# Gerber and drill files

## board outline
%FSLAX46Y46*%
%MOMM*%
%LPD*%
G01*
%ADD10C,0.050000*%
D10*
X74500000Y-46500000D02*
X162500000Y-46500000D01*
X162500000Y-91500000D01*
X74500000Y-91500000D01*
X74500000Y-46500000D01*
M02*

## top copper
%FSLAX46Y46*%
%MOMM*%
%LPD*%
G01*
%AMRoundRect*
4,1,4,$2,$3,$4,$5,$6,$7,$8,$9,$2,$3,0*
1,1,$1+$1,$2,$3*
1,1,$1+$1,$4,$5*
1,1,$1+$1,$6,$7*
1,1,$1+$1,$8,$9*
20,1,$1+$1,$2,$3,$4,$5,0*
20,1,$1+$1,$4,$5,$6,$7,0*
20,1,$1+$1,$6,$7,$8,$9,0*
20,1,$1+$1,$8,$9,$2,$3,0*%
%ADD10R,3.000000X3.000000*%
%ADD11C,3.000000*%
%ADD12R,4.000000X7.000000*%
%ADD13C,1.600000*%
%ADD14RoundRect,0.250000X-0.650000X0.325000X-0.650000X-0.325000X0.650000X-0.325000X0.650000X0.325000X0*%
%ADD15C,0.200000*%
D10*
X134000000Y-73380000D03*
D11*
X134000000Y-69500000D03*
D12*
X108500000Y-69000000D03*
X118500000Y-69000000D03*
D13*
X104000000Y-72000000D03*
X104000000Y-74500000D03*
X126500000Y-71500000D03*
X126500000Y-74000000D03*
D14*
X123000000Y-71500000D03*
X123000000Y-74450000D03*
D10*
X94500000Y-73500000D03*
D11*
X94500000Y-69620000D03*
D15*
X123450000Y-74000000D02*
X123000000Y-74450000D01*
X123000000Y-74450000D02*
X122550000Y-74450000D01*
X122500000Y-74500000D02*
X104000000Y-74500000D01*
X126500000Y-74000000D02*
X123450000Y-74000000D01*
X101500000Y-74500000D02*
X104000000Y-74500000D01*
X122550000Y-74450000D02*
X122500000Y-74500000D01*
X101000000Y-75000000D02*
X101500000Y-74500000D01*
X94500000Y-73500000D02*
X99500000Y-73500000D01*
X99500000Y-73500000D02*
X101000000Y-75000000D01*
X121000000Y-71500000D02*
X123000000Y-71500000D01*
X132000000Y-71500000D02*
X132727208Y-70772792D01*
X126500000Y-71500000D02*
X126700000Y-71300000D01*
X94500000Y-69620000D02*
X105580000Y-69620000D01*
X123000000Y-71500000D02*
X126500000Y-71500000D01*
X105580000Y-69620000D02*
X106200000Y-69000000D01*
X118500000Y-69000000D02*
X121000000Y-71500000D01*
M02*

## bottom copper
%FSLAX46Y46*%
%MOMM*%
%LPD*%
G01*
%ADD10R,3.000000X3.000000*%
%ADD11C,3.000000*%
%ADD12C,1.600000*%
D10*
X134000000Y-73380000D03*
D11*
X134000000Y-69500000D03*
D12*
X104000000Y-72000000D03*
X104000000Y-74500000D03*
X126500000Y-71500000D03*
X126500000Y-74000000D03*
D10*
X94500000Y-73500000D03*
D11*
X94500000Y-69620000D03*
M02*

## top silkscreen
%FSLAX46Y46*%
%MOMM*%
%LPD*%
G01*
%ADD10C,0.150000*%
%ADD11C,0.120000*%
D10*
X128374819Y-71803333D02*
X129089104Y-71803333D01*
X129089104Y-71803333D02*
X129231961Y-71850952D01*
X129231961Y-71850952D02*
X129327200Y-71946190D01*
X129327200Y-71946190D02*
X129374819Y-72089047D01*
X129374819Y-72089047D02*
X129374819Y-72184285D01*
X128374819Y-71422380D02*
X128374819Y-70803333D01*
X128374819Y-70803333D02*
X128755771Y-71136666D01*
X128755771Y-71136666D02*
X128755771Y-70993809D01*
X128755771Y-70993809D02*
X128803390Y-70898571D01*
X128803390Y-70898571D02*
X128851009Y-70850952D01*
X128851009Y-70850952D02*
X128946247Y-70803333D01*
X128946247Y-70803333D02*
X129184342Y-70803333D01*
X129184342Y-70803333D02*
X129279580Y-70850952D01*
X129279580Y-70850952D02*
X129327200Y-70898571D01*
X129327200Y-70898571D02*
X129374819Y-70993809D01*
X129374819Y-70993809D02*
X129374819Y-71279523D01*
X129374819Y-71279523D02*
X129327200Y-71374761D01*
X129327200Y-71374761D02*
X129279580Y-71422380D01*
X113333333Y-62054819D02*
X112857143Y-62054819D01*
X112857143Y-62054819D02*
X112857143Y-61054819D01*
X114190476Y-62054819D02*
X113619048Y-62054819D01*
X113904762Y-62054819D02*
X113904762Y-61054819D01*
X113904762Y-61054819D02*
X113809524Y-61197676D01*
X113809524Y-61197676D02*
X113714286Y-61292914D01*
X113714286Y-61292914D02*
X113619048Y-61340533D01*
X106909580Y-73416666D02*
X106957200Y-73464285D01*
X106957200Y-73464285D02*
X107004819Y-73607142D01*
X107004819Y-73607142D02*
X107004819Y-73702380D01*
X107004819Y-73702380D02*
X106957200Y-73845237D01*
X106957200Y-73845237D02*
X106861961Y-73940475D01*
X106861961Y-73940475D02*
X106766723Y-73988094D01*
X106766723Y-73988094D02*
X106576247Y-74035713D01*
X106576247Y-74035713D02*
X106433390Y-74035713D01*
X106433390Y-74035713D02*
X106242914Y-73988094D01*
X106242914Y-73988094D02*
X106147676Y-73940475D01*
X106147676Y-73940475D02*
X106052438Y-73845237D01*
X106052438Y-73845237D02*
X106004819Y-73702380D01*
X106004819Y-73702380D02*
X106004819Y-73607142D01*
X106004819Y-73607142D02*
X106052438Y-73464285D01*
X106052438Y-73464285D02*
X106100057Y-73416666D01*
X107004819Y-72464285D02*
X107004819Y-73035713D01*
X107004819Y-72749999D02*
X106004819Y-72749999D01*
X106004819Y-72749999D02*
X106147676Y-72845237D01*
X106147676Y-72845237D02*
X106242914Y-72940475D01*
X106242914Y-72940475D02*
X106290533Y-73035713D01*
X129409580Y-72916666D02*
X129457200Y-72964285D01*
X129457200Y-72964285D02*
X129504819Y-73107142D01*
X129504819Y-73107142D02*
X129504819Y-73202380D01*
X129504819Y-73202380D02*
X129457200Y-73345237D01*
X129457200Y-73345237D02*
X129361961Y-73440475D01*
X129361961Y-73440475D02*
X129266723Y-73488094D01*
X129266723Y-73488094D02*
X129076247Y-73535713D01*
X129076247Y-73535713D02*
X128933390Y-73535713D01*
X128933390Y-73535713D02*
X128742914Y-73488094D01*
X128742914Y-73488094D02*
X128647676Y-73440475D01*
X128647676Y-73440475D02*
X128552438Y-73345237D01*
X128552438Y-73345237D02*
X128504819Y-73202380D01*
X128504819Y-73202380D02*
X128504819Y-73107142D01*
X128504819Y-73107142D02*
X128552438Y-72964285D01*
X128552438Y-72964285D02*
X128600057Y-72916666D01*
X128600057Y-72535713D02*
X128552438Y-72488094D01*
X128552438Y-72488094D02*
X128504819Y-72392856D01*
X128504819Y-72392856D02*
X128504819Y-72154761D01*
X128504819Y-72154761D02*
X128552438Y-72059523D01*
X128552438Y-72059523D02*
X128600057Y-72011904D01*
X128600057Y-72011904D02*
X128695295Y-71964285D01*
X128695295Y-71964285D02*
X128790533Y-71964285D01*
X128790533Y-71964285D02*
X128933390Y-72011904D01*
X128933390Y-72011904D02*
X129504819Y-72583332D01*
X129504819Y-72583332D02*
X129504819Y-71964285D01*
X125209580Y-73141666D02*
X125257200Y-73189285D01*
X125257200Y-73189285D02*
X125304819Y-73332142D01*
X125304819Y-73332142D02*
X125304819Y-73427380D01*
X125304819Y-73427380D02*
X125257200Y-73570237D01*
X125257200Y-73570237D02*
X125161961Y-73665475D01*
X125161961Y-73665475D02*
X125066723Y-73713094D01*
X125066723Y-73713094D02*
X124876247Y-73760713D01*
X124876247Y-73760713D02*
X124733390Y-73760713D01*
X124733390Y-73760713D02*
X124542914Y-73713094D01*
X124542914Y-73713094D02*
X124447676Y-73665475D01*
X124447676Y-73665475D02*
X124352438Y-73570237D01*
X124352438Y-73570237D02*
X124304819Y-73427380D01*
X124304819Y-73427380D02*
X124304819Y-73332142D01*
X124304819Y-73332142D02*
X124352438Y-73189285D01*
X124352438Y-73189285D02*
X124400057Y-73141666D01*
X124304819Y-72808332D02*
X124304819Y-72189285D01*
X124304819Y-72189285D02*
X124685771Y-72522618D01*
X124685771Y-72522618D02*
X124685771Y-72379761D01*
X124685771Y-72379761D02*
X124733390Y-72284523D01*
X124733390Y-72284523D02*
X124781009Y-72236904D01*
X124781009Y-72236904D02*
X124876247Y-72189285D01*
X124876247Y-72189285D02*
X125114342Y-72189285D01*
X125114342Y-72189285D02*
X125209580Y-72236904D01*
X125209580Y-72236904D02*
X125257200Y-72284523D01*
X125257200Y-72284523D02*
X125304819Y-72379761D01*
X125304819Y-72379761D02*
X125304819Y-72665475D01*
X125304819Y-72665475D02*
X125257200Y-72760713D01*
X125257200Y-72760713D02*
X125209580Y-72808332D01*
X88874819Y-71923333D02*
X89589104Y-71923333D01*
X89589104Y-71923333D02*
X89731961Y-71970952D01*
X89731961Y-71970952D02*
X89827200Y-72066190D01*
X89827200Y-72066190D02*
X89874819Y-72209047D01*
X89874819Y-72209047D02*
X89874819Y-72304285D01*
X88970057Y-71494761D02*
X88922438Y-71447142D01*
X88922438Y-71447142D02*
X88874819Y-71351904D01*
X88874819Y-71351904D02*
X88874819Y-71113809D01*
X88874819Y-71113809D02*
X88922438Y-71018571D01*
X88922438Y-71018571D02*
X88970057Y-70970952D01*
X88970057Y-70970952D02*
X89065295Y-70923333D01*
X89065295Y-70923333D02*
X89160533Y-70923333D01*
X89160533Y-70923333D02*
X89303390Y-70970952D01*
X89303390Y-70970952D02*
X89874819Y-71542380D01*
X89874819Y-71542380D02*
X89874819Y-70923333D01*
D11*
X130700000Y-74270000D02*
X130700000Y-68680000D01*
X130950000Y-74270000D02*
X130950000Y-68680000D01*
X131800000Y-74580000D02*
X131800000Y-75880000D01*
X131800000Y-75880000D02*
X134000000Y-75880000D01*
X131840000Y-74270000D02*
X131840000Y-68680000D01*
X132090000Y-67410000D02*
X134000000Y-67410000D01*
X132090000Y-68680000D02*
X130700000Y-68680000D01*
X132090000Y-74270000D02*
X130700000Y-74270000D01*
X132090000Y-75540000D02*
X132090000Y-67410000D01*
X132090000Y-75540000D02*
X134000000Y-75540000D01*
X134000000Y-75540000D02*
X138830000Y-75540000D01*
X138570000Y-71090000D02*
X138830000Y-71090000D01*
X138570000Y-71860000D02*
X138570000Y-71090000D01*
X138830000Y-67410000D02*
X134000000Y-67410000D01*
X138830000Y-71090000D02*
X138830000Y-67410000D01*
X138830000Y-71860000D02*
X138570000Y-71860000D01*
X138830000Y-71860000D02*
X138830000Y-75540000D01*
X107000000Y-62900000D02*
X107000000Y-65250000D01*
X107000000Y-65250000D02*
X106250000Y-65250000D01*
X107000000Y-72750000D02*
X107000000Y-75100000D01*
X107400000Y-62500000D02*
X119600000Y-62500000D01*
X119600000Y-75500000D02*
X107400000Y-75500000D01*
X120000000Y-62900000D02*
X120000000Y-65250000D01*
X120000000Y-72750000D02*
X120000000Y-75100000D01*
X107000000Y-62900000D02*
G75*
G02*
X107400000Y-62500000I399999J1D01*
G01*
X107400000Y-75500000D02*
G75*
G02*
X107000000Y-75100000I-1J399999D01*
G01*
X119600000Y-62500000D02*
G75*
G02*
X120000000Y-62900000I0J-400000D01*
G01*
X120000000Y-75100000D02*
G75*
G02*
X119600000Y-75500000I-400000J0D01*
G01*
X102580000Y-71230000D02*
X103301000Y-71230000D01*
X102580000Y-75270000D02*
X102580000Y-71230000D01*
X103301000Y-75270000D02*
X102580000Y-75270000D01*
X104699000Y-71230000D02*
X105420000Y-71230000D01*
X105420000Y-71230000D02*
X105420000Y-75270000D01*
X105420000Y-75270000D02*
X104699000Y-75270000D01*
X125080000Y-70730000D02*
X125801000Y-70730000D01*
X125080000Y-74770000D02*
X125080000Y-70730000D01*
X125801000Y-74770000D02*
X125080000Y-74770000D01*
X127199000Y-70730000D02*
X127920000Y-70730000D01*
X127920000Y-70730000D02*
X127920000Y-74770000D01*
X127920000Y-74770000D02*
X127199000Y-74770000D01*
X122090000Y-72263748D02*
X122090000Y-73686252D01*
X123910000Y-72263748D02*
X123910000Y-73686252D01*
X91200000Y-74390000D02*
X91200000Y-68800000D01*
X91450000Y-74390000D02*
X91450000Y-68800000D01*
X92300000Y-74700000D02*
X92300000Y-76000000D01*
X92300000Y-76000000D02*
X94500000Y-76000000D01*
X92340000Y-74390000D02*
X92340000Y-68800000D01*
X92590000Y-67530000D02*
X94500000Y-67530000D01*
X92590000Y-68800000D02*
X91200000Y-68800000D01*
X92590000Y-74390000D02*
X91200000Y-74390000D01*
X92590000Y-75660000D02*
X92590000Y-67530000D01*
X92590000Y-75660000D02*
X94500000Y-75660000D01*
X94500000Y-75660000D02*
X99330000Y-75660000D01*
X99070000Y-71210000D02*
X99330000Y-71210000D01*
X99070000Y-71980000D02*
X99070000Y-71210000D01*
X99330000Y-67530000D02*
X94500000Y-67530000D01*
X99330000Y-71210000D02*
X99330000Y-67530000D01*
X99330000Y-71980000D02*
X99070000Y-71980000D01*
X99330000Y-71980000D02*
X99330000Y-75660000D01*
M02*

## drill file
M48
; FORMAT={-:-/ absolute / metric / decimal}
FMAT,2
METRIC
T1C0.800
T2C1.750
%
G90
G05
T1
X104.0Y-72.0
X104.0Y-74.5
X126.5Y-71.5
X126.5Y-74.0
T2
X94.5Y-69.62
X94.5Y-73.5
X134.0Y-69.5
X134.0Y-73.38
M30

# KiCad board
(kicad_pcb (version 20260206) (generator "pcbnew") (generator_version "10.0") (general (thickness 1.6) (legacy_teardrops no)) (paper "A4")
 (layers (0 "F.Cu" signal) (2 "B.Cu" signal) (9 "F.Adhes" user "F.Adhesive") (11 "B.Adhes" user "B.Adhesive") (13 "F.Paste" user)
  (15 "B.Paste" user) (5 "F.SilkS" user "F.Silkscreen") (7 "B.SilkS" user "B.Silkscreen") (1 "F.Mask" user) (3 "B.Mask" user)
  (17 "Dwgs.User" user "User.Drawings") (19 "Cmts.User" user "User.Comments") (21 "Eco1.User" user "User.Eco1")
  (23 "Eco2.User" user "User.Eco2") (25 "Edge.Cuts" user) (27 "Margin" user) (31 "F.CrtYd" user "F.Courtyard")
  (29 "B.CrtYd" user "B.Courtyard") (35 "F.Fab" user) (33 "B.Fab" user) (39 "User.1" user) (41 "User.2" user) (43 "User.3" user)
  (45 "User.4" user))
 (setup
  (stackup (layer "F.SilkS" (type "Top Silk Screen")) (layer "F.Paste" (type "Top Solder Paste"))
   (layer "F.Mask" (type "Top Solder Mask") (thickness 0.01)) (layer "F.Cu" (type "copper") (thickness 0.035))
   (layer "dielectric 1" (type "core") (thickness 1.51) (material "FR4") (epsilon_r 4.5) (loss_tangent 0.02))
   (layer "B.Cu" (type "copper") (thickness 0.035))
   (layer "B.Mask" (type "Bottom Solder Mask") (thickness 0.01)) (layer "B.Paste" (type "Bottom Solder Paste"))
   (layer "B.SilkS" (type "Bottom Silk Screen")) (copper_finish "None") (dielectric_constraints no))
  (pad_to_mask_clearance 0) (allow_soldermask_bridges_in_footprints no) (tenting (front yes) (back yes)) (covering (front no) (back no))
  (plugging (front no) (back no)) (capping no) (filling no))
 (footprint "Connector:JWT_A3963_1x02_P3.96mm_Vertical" (layer "F.Cu") (at 134 73.38 90)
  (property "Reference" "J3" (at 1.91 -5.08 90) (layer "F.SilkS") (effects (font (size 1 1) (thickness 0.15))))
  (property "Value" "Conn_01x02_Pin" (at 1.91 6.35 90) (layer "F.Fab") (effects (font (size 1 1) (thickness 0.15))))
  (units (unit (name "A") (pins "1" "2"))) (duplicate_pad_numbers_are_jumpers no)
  (fp_line (start -0.89 -3.3) (end 4.7 -3.3) (stroke (width 0.12) (type solid)) (layer "F.SilkS"))
  (fp_line (start -0.89 -3.05) (end 4.7 -3.05) (stroke (width 0.12) (type solid)) (layer "F.SilkS"))
  (fp_line (start -1.2 -2.2) (end -2.5 -2.2) (stroke (width 0.12) (type solid)) (layer "F.SilkS"))
  (fp_line (start -2.5 -2.2) (end -2.5 0) (stroke (width 0.12) (type solid)) (layer "F.SilkS"))
  (fp_line (start -0.89 -2.16) (end 4.7 -2.16) (stroke (width 0.12) (type solid)) (layer "F.SilkS"))
  (fp_line (start 5.97 -1.91) (end 5.97 0) (stroke (width 0.12) (type solid)) (layer "F.SilkS"))
  (fp_line (start 4.7 -1.91) (end 4.7 -3.3) (stroke (width 0.12) (type solid)) (layer "F.SilkS"))
  (fp_line (start -0.89 -1.91) (end -0.89 -3.3) (stroke (width 0.12) (type solid)) (layer "F.SilkS"))
  (fp_line (start -2.16 -1.91) (end 5.97 -1.91) (stroke (width 0.12) (type solid)) (layer "F.SilkS"))
  (fp_line (start -2.16 -1.91) (end -2.16 0) (stroke (width 0.12) (type solid)) (layer "F.SilkS"))
  (fp_line (start -2.16 0) (end -2.16 4.83) (stroke (width 0.12) (type solid)) (layer "F.SilkS"))
  (fp_line (start 2.29 4.57) (end 2.29 4.83) (stroke (width 0.12) (type solid)) (layer "F.SilkS"))
  (fp_line (start 1.52 4.57) (end 2.29 4.57) (stroke (width 0.12) (type solid)) (layer "F.SilkS"))
  (fp_line (start 5.97 4.83) (end 5.97 0) (stroke (width 0.12) (type solid)) (layer "F.SilkS"))
  (fp_line (start 2.29 4.83) (end 5.97 4.83) (stroke (width 0.12) (type solid)) (layer "F.SilkS"))
  (fp_line (start 1.52 4.83) (end 1.52 4.57) (stroke (width 0.12) (type solid)) (layer "F.SilkS"))
  (fp_line (start 1.52 4.83) (end -2.16 4.83) (stroke (width 0.12) (type solid)) (layer "F.SilkS"))
  (pad "1" thru_hole rect (at 0 0 90) (size 3 3) (drill 1.75) (layers "*.Cu" "*.Mask") (remove_unused_layers no) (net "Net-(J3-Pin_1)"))
  (pad "2" thru_hole circle (at 3.88 0 90) (size 3 3) (drill 1.75) (layers "*.Cu" "*.Mask") (remove_unused_layers no) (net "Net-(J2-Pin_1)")))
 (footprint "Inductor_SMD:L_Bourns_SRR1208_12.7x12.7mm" (layer "F.Cu") (at 113.5 69)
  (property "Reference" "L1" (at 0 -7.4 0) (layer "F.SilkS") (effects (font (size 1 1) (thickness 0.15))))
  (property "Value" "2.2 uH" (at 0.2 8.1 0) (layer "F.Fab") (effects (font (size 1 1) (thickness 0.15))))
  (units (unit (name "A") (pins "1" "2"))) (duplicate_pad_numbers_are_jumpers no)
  (fp_line (start -6.5 -6.1) (end -6.5 -3.75) (stroke (width 0.12) (type solid)) (layer "F.SilkS"))
  (fp_line (start -6.5 -3.75) (end -7.25 -3.75) (stroke (width 0.12) (type solid)) (layer "F.SilkS"))
  (fp_line (start -6.5 3.75) (end -6.5 6.1) (stroke (width 0.12) (type solid)) (layer "F.SilkS"))
  (fp_line (start -6.1 -6.5) (end 6.1 -6.5) (stroke (width 0.12) (type solid)) (layer "F.SilkS"))
  (fp_line (start 6.1 6.5) (end -6.1 6.5) (stroke (width 0.12) (type solid)) (layer "F.SilkS"))
  (fp_line (start 6.5 -6.1) (end 6.5 -3.75) (stroke (width 0.12) (type solid)) (layer "F.SilkS"))
  (fp_line (start 6.5 3.75) (end 6.5 6.1) (stroke (width 0.12) (type solid)) (layer "F.SilkS"))
  (fp_arc (start -6.5 -6.1) (mid -6.382843 -6.382843) (end -6.1 -6.5) (stroke (width 0.12) (type solid)) (layer "F.SilkS"))
  (fp_arc (start -6.1 6.5) (mid -6.382843 6.382843) (end -6.5 6.1) (stroke (width 0.12) (type solid)) (layer "F.SilkS"))
  (fp_arc (start 6.1 -6.5) (mid 6.382843 -6.382843) (end 6.5 -6.1) (stroke (width 0.12) (type solid)) (layer "F.SilkS"))
  (fp_arc (start 6.5 6.1) (mid 6.382843 6.382843) (end 6.1 6.5) (stroke (width 0.12) (type solid)) (layer "F.SilkS"))
  (pad "1" smd rect (at -5 0) (size 4 7) (layers "F.Cu" "F.Mask" "F.Paste") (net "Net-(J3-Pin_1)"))
  (pad "2" smd rect (at 5 0) (size 4 7) (layers "F.Cu" "F.Mask" "F.Paste") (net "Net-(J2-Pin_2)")))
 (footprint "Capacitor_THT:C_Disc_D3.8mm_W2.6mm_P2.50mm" (layer "F.Cu") (at 104 72 -90)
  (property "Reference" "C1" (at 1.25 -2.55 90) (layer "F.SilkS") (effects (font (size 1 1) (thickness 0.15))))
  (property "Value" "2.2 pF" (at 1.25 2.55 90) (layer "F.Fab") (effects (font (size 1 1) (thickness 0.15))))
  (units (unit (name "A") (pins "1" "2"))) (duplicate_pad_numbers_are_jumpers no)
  (fp_line (start -0.77 1.42) (end -0.77 0.699) (stroke (width 0.12) (type solid)) (layer "F.SilkS"))
  (fp_line (start 3.27 1.42) (end -0.77 1.42) (stroke (width 0.12) (type solid)) (layer "F.SilkS"))
  (fp_line (start 3.27 0.699) (end 3.27 1.42) (stroke (width 0.12) (type solid)) (layer "F.SilkS"))
  (fp_line (start -0.77 -0.699) (end -0.77 -1.42) (stroke (width 0.12) (type solid)) (layer "F.SilkS"))
  (fp_line (start -0.77 -1.42) (end 3.27 -1.42) (stroke (width 0.12) (type solid)) (layer "F.SilkS"))
  (fp_line (start 3.27 -1.42) (end 3.27 -0.699) (stroke (width 0.12) (type solid)) (layer "F.SilkS"))
  (pad "1" thru_hole circle (at 0 0 270) (size 1.6 1.6) (drill 0.8) (layers "*.Cu" "*.Mask") (remove_unused_layers no)
   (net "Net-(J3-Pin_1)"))
  (pad "2" thru_hole circle (at 2.5 0 270) (size 1.6 1.6) (drill 0.8) (layers "*.Cu" "*.Mask") (remove_unused_layers no)
   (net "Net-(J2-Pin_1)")))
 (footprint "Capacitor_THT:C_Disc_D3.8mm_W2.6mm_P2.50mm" (layer "F.Cu") (at 126.5 71.5 -90)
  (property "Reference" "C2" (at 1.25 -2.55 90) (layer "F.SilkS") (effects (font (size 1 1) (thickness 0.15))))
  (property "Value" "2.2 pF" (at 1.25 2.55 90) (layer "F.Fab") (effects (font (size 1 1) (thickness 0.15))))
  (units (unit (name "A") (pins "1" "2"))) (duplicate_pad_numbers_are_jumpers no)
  (fp_line (start -0.77 1.42) (end -0.77 0.699) (stroke (width 0.12) (type solid)) (layer "F.SilkS"))
  (fp_line (start 3.27 1.42) (end -0.77 1.42) (stroke (width 0.12) (type solid)) (layer "F.SilkS"))
  (fp_line (start 3.27 0.699) (end 3.27 1.42) (stroke (width 0.12) (type solid)) (layer "F.SilkS"))
  (fp_line (start -0.77 -0.699) (end -0.77 -1.42) (stroke (width 0.12) (type solid)) (layer "F.SilkS"))
  (fp_line (start -0.77 -1.42) (end 3.27 -1.42) (stroke (width 0.12) (type solid)) (layer "F.SilkS"))
  (fp_line (start 3.27 -1.42) (end 3.27 -0.699) (stroke (width 0.12) (type solid)) (layer "F.SilkS"))
  (pad "1" thru_hole circle (at 0 0 270) (size 1.6 1.6) (drill 0.8) (layers "*.Cu" "*.Mask") (remove_unused_layers no)
   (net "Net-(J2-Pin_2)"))
  (pad "2" thru_hole circle (at 2.5 0 270) (size 1.6 1.6) (drill 0.8) (layers "*.Cu" "*.Mask") (remove_unused_layers no)
   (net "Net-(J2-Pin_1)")))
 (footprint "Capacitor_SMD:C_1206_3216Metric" (layer "F.Cu") (at 123 72.975 -90)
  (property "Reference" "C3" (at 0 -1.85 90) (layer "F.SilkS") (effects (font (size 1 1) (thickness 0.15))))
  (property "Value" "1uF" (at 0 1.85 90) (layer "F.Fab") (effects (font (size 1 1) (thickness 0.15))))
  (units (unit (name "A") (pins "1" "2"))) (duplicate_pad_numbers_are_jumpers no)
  (fp_line (start -0.711252 0.91) (end 0.711252 0.91) (stroke (width 0.12) (type solid)) (layer "F.SilkS"))
  (fp_line (start -0.711252 -0.91) (end 0.711252 -0.91) (stroke (width 0.12) (type solid)) (layer "F.SilkS"))
  (pad "1" smd roundrect (at -1.475 0 270) (size 1.15 1.8) (layers "F.Cu" "F.Mask" "F.Paste") (roundrect_rratio 0.217391)
   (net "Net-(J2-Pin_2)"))
  (pad "2" smd roundrect (at 1.475 0 270) (size 1.15 1.8) (layers "F.Cu" "F.Mask" "F.Paste") (roundrect_rratio 0.217391)
   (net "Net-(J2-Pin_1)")))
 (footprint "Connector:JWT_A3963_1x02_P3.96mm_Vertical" (layer "F.Cu") (at 94.5 73.5 90)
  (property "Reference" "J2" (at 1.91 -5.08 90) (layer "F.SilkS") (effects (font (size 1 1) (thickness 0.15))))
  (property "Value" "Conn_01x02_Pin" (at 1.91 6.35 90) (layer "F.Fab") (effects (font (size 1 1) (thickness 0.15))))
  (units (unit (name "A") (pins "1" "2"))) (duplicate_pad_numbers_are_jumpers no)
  (fp_line (start -0.89 -3.3) (end 4.7 -3.3) (stroke (width 0.12) (type solid)) (layer "F.SilkS"))
  (fp_line (start -0.89 -3.05) (end 4.7 -3.05) (stroke (width 0.12) (type solid)) (layer "F.SilkS"))
  (fp_line (start -1.2 -2.2) (end -2.5 -2.2) (stroke (width 0.12) (type solid)) (layer "F.SilkS"))
  (fp_line (start -2.5 -2.2) (end -2.5 0) (stroke (width 0.12) (type solid)) (layer "F.SilkS"))
  (fp_line (start -0.89 -2.16) (end 4.7 -2.16) (stroke (width 0.12) (type solid)) (layer "F.SilkS"))
  (fp_line (start 5.97 -1.91) (end 5.97 0) (stroke (width 0.12) (type solid)) (layer "F.SilkS"))
  (fp_line (start 4.7 -1.91) (end 4.7 -3.3) (stroke (width 0.12) (type solid)) (layer "F.SilkS"))
  (fp_line (start -0.89 -1.91) (end -0.89 -3.3) (stroke (width 0.12) (type solid)) (layer "F.SilkS"))
  (fp_line (start -2.16 -1.91) (end 5.97 -1.91) (stroke (width 0.12) (type solid)) (layer "F.SilkS"))
  (fp_line (start -2.16 -1.91) (end -2.16 0) (stroke (width 0.12) (type solid)) (layer "F.SilkS"))
  (fp_line (start -2.16 0) (end -2.16 4.83) (stroke (width 0.12) (type solid)) (layer "F.SilkS"))
  (fp_line (start 2.29 4.57) (end 2.29 4.83) (stroke (width 0.12) (type solid)) (layer "F.SilkS"))
  (fp_line (start 1.52 4.57) (end 2.29 4.57) (stroke (width 0.12) (type solid)) (layer "F.SilkS"))
  (fp_line (start 5.97 4.83) (end 5.97 0) (stroke (width 0.12) (type solid)) (layer "F.SilkS"))
  (fp_line (start 2.29 4.83) (end 5.97 4.83) (stroke (width 0.12) (type solid)) (layer "F.SilkS"))
  (fp_line (start 1.52 4.83) (end 1.52 4.57) (stroke (width 0.12) (type solid)) (layer "F.SilkS"))
  (fp_line (start 1.52 4.83) (end -2.16 4.83) (stroke (width 0.12) (type solid)) (layer "F.SilkS"))
  (pad "1" thru_hole rect (at 0 0 90) (size 3 3) (drill 1.75) (layers "*.Cu" "*.Mask") (remove_unused_layers no) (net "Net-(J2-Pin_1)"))
  (pad "2" thru_hole circle (at 3.88 0 90) (size 3 3) (drill 1.75) (layers "*.Cu" "*.Mask") (remove_unused_layers no) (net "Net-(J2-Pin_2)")))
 (gr_rect (start 74.5 46.5) (end 162.5 91.5) (stroke (width 0.05) (type default)) (fill no) (layer "Edge.Cuts"))
 (segment (start 123.45 74) (end 123 74.45) (width 0.2) (layer "F.Cu") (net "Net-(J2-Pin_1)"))
 (segment (start 123 74.45) (end 122.55 74.45) (width 0.2) (layer "F.Cu") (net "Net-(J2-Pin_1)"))
 (segment (start 122.5 74.5) (end 104 74.5) (width 0.2) (layer "F.Cu") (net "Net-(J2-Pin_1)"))
 (segment (start 126.5 74) (end 123.45 74) (width 0.2) (layer "F.Cu") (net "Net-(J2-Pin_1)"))
 (segment (start 101.5 74.5) (end 104 74.5) (width 0.2) (layer "F.Cu") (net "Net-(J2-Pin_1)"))
 (segment (start 122.55 74.45) (end 122.5 74.5) (width 0.2) (layer "F.Cu") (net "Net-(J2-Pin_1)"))
 (segment (start 101 75) (end 101.5 74.5) (width 0.2) (layer "F.Cu") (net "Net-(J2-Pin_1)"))
 (segment (start 94.5 73.5) (end 99.5 73.5) (width 0.2) (layer "F.Cu") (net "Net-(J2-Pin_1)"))
 (segment (start 99.5 73.5) (end 101 75) (width 0.2) (layer "F.Cu") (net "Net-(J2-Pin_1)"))
 (segment (start 121 71.5) (end 123 71.5) (width 0.2) (layer "F.Cu") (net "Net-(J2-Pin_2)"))
 (segment (start 132 71.5) (end 132.727208 70.772792) (width 0.2) (layer "F.Cu") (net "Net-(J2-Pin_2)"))
 (segment (start 126.5 71.5) (end 126.7 71.3) (width 0.2) (layer "F.Cu") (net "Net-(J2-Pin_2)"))
 (segment (start 94.5 69.62) (end 105.58 69.62) (width 0.2) (layer "F.Cu") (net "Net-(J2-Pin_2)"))
 (segment (start 123 71.5) (end 126.5 71.5) (width 0.2) (layer "F.Cu") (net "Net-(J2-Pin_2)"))
 (segment (start 105.58 69.62) (end 106.2 69) (width 0.2) (layer "F.Cu") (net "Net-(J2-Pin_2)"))
 (segment (start 118.5 69) (end 121 71.5) (width 0.2) (layer "F.Cu") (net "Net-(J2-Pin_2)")))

